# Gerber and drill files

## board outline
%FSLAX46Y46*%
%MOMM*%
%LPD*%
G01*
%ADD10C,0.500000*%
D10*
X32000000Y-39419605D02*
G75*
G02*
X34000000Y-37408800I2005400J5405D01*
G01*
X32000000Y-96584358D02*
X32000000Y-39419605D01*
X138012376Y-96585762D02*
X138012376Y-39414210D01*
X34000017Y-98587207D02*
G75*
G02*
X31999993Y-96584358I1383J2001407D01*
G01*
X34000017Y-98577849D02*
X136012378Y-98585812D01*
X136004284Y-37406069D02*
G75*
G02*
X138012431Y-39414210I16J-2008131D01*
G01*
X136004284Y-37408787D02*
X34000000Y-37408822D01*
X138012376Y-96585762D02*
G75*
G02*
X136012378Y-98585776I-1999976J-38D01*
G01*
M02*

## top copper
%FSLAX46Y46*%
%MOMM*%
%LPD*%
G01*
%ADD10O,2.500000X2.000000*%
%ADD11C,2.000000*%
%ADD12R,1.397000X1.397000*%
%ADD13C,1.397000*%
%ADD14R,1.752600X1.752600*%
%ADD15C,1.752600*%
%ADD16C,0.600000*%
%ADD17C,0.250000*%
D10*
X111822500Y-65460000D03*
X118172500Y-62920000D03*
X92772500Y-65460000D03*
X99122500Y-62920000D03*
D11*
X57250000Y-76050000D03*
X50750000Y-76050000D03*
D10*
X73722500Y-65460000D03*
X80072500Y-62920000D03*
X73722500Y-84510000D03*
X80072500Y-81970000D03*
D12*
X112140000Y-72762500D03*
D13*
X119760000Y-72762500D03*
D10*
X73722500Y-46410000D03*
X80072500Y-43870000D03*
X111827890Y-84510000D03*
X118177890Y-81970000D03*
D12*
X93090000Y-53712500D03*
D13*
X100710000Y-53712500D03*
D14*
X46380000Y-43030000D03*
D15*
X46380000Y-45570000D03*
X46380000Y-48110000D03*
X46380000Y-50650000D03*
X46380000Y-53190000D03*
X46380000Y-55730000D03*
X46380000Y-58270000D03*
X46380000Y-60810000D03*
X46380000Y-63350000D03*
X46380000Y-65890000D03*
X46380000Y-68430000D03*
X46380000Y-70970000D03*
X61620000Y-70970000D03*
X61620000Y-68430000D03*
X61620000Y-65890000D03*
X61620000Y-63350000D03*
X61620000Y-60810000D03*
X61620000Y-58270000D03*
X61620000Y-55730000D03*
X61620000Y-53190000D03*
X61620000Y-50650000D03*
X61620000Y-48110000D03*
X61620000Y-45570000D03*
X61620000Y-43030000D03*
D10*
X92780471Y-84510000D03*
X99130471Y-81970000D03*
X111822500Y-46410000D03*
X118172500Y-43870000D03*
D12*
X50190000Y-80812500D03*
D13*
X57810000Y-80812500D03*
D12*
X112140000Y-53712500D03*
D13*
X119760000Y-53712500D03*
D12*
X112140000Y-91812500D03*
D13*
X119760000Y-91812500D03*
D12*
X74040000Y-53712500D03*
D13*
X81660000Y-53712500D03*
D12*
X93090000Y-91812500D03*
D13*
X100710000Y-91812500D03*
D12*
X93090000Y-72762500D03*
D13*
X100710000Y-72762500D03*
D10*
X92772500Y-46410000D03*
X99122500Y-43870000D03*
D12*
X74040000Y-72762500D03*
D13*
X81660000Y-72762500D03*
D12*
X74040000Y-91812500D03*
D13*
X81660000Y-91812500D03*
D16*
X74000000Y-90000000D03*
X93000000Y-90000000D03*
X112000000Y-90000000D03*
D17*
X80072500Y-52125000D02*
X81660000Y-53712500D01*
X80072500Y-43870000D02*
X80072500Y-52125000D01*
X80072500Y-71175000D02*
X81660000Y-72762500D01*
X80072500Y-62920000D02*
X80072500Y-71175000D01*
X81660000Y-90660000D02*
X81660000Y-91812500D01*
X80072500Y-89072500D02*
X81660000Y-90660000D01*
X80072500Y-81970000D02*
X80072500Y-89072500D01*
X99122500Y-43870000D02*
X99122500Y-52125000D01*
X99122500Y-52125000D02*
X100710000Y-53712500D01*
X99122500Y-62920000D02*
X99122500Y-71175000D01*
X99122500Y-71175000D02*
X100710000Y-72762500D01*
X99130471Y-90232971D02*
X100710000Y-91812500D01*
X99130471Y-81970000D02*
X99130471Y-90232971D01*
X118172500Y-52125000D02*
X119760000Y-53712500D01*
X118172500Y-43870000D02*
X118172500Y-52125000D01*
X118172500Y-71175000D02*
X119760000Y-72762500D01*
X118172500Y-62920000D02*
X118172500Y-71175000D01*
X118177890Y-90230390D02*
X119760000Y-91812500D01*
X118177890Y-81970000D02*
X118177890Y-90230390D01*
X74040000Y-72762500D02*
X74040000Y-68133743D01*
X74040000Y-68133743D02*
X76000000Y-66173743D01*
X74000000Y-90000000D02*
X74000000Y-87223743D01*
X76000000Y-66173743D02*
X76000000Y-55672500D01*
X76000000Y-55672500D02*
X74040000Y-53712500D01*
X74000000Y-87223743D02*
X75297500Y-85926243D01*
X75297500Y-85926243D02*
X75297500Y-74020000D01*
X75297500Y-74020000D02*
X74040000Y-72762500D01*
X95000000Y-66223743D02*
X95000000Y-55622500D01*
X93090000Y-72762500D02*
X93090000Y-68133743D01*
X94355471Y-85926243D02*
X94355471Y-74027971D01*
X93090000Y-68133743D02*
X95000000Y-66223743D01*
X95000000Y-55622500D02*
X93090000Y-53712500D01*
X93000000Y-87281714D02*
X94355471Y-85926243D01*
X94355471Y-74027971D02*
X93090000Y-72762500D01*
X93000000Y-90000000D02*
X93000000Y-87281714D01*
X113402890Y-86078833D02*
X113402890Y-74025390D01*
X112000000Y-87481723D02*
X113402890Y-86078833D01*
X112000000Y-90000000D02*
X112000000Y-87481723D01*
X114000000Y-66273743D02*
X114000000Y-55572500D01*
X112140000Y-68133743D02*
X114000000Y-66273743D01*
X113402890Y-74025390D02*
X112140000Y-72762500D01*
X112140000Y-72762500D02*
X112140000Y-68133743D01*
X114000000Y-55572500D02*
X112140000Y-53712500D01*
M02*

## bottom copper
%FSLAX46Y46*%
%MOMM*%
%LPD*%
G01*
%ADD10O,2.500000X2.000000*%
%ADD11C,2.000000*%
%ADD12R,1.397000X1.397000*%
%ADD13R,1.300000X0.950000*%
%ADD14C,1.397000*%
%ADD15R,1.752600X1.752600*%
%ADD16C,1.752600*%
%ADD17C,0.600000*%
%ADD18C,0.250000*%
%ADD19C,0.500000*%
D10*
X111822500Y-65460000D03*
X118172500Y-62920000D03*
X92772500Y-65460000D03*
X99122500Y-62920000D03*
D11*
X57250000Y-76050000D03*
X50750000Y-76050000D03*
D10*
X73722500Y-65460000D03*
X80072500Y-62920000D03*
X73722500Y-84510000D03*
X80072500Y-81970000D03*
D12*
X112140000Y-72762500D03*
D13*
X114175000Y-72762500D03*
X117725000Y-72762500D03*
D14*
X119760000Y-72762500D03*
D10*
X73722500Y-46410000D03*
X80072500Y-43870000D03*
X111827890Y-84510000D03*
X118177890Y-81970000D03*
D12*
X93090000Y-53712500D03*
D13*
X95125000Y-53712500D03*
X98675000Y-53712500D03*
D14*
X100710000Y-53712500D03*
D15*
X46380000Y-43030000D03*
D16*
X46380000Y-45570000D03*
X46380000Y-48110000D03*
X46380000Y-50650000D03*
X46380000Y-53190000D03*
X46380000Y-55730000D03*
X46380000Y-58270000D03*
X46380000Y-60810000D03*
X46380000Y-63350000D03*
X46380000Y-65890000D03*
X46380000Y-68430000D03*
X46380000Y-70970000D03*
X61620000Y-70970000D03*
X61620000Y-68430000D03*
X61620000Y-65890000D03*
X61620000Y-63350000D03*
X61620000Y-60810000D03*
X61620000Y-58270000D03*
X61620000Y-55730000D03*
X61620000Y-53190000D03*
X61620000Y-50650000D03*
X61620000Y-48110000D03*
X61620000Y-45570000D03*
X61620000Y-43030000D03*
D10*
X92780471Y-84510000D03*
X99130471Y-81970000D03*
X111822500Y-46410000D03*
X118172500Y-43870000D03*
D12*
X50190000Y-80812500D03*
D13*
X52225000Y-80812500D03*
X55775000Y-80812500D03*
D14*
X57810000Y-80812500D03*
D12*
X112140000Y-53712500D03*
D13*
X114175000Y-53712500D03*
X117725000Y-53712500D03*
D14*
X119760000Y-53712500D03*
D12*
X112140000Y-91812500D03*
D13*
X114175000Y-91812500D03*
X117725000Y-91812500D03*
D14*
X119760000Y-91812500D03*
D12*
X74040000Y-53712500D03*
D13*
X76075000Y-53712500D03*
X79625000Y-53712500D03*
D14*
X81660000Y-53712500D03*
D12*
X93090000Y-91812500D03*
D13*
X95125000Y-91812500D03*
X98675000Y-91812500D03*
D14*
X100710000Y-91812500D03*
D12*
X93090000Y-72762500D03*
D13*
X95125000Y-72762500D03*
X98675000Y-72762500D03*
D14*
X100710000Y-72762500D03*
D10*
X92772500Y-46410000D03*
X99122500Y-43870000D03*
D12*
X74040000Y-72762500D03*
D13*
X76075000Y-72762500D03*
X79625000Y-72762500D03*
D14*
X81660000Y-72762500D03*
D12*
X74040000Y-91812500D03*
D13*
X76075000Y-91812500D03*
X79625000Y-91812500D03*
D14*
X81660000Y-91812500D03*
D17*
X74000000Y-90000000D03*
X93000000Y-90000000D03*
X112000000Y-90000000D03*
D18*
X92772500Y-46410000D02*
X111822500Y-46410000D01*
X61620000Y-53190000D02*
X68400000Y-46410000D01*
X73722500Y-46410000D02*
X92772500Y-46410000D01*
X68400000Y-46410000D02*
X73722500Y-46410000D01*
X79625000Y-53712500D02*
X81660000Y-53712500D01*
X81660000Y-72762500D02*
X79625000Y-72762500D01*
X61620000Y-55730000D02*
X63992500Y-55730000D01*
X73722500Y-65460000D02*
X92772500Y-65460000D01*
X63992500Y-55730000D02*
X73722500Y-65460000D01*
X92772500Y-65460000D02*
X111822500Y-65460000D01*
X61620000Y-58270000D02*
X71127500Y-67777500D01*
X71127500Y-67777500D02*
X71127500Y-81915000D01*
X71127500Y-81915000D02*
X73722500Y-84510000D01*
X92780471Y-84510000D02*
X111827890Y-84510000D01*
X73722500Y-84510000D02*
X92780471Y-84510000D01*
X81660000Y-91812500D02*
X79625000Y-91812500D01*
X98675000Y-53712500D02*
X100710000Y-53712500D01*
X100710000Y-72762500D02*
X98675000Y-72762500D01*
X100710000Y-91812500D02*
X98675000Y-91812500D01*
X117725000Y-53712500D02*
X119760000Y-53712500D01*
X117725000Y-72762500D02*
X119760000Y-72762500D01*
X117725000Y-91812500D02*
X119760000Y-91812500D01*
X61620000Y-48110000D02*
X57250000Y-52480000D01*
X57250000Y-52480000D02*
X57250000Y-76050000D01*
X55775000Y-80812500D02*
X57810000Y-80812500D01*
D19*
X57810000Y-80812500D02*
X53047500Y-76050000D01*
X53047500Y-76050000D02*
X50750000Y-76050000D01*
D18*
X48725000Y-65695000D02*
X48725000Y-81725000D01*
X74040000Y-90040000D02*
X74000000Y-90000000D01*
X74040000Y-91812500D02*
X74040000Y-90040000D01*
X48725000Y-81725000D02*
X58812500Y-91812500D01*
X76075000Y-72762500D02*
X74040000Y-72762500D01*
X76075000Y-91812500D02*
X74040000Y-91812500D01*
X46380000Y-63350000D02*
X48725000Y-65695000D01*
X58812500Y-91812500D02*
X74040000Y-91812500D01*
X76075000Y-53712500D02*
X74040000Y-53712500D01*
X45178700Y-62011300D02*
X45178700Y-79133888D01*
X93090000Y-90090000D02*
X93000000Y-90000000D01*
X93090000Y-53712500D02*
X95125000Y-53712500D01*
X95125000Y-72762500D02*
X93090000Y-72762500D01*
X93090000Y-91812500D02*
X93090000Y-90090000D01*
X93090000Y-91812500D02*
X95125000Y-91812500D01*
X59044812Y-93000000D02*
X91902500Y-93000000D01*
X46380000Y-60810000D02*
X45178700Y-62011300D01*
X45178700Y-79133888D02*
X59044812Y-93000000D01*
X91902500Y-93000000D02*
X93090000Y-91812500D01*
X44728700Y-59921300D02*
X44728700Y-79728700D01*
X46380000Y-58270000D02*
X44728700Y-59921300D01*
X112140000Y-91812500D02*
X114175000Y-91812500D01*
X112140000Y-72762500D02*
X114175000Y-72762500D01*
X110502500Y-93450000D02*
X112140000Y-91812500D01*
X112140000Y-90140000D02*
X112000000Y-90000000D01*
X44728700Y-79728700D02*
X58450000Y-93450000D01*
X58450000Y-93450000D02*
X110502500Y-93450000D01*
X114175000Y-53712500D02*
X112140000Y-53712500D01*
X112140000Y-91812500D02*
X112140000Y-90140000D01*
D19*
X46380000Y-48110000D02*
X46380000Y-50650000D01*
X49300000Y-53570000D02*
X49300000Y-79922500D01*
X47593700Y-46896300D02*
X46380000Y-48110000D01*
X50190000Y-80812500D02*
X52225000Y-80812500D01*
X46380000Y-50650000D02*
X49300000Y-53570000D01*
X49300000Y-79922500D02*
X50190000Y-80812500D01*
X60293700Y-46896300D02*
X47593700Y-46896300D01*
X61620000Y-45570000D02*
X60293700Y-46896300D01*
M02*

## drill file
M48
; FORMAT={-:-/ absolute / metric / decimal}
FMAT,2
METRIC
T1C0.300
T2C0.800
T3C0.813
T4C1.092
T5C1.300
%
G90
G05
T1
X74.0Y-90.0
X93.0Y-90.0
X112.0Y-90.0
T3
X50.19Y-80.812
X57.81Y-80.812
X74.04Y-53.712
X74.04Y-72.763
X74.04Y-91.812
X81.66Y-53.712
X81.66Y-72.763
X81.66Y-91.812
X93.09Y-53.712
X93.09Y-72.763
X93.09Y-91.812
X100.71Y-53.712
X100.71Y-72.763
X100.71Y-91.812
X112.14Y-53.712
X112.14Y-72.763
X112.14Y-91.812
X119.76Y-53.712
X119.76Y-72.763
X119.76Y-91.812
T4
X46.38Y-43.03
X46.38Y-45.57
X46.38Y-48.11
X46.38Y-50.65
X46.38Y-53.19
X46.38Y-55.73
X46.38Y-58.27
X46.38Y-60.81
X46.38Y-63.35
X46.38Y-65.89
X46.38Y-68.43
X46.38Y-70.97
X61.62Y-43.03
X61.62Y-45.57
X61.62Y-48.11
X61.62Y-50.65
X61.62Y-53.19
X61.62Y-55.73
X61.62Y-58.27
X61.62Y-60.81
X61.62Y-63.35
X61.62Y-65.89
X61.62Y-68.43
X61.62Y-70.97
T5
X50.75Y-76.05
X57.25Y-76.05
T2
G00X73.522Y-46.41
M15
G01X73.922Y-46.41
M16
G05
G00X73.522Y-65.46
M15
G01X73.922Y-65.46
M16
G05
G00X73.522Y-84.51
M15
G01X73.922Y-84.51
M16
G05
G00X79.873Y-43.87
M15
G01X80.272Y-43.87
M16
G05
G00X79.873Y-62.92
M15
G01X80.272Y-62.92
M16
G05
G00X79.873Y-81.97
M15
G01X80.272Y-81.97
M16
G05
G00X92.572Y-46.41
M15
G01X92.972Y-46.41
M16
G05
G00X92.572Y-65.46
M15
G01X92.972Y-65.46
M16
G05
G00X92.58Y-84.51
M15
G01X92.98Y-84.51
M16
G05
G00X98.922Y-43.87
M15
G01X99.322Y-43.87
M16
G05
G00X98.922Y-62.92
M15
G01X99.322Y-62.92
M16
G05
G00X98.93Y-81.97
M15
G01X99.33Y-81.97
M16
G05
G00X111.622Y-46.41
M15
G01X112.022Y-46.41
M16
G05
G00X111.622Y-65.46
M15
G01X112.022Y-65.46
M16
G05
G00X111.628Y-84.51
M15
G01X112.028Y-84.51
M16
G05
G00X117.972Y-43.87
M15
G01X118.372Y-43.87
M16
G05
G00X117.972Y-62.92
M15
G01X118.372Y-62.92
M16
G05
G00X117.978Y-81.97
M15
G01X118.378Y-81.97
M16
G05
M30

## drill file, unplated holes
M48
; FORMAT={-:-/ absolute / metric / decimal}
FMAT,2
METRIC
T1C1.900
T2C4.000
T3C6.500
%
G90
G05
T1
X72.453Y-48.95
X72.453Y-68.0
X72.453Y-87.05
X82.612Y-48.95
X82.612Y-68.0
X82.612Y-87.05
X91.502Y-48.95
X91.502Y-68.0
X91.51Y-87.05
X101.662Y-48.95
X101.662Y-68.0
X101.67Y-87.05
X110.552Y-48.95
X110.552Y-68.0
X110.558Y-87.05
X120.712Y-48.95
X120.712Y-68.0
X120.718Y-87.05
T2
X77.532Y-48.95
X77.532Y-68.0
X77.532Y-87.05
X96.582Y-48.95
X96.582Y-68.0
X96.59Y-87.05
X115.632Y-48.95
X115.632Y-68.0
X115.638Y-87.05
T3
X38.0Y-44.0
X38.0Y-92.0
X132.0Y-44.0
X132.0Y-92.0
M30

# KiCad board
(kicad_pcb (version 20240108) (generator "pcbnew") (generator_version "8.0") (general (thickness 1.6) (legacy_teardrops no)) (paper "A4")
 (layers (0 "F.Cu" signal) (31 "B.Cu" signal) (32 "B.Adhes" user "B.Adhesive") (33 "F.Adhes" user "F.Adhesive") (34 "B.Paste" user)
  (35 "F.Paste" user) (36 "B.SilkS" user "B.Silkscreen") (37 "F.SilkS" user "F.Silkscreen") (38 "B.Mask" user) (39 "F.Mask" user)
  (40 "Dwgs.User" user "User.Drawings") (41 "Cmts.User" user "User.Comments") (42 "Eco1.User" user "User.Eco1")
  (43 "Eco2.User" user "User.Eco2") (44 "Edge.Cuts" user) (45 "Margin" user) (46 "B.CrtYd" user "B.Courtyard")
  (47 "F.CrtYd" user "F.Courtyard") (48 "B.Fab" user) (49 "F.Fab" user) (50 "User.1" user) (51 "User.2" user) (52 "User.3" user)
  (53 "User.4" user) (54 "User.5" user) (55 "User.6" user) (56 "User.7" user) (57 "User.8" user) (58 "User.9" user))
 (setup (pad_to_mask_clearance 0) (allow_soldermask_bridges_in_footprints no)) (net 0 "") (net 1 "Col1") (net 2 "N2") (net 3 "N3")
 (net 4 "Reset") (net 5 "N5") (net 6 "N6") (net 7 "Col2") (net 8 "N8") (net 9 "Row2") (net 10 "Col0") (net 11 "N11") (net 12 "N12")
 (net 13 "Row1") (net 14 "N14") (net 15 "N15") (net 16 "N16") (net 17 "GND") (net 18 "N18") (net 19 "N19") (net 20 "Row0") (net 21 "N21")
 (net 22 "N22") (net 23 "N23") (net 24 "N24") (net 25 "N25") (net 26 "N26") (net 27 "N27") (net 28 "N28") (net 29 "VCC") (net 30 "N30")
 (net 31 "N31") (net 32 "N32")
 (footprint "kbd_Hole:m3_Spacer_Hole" (layer "F.Cu") (at 38 92)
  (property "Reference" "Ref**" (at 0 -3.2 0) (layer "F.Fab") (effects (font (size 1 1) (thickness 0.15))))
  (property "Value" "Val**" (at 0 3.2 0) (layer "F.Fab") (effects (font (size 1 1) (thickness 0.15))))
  (pad "" np_thru_hole circle (at 0 0) (size 6.5 6.5) (drill 6.5) (layers "*.Cu" "*.Mask")))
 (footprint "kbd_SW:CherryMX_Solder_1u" (layer "F.Cu") (at 115.6325 68)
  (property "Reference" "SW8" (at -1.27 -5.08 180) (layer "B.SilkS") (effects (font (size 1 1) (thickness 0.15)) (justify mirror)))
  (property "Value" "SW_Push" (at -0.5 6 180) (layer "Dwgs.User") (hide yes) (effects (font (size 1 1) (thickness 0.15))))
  (pad "" np_thru_hole circle (at -5.08 0 90) (size 1.9 1.9) (drill 1.9) (layers "*.Cu" "*.Mask"))
  (pad "" np_thru_hole circle (at 0 0 90) (size 4 4) (drill 4) (layers "*.Cu" "*.Mask"))
  (pad "" np_thru_hole circle (at 5.08 0 90) (size 1.9 1.9) (drill 1.9) (layers "*.Cu" "*.Mask"))
  (pad "1" thru_hole oval (at -3.81 -2.54) (size 2.5 2) (drill oval 1.2 0.8) (layers "*.Cu" "F.SilkS" "B.Mask") (remove_unused_layers no)
   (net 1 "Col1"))
  (pad "2" thru_hole oval (at 2.54 -5.08) (size 2.5 2) (drill oval 1.2 0.8) (layers "*.Cu" "F.SilkS" "B.Mask") (remove_unused_layers no)
   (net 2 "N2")))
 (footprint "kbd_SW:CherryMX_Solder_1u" (layer "F.Cu") (at 96.5825 68)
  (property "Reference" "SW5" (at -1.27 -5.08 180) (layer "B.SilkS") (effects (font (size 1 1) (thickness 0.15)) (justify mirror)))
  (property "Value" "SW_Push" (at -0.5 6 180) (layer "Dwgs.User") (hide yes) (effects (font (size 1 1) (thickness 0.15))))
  (pad "" np_thru_hole circle (at -5.08 0 90) (size 1.9 1.9) (drill 1.9) (layers "*.Cu" "*.Mask"))
  (pad "" np_thru_hole circle (at 0 0 90) (size 4 4) (drill 4) (layers "*.Cu" "*.Mask"))
  (pad "" np_thru_hole circle (at 5.08 0 90) (size 1.9 1.9) (drill 1.9) (layers "*.Cu" "*.Mask"))
  (pad "1" thru_hole oval (at -3.81 -2.54) (size 2.5 2) (drill oval 1.2 0.8) (layers "*.Cu" "F.SilkS" "B.Mask") (remove_unused_layers no)
   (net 1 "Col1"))
  (pad "2" thru_hole oval (at 2.54 -5.08) (size 2.5 2) (drill oval 1.2 0.8) (layers "*.Cu" "F.SilkS" "B.Mask") (remove_unused_layers no)
   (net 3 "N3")))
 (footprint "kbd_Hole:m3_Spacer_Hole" (layer "F.Cu") (at 132 92)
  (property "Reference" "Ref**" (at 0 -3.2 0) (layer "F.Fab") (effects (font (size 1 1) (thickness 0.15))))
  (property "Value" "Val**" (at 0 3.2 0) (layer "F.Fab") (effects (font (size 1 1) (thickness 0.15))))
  (pad "" np_thru_hole circle (at 0 0) (size 6.5 6.5) (drill 6.5) (layers "*.Cu" "*.Mask")))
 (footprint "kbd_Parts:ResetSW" (layer "F.Cu") (at 54 76.05)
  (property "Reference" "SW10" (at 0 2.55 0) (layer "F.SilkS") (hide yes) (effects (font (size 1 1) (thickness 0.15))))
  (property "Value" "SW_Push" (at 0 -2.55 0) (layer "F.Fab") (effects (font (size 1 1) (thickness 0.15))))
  (pad "1" thru_hole circle (at 3.25 0) (size 2 2) (drill 1.3) (layers "*.Cu" "*.Mask" "F.SilkS") (remove_unused_layers no) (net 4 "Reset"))
  (pad "2" thru_hole circle (at -3.25 0) (size 2 2) (drill 1.3) (layers "*.Cu" "*.Mask" "F.SilkS") (remove_unused_layers no) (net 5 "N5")))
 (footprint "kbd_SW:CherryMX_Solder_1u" (layer "F.Cu") (at 77.5325 68)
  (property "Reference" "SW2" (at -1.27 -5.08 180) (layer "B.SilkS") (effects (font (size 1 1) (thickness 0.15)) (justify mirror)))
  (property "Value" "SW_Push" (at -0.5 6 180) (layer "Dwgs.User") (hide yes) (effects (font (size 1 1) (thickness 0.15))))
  (pad "" np_thru_hole circle (at -5.08 0 90) (size 1.9 1.9) (drill 1.9) (layers "*.Cu" "*.Mask"))
  (pad "" np_thru_hole circle (at 0 0 90) (size 4 4) (drill 4) (layers "*.Cu" "*.Mask"))
  (pad "" np_thru_hole circle (at 5.08 0 90) (size 1.9 1.9) (drill 1.9) (layers "*.Cu" "*.Mask"))
  (pad "1" thru_hole oval (at -3.81 -2.54) (size 2.5 2) (drill oval 1.2 0.8) (layers "*.Cu" "F.SilkS" "B.Mask") (remove_unused_layers no)
   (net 1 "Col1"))
  (pad "2" thru_hole oval (at 2.54 -5.08) (size 2.5 2) (drill oval 1.2 0.8) (layers "*.Cu" "F.SilkS" "B.Mask") (remove_unused_layers no)
   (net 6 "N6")))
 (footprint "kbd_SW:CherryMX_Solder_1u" (layer "F.Cu") (at 77.5325 87.05)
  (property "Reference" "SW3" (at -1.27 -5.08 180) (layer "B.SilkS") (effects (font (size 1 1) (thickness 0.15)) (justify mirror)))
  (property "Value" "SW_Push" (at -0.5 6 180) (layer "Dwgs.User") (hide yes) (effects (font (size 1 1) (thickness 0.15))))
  (pad "" np_thru_hole circle (at -5.08 0 90) (size 1.9 1.9) (drill 1.9) (layers "*.Cu" "*.Mask"))
  (pad "" np_thru_hole circle (at 0 0 90) (size 4 4) (drill 4) (layers "*.Cu" "*.Mask"))
  (pad "" np_thru_hole circle (at 5.08 0 90) (size 1.9 1.9) (drill 1.9) (layers "*.Cu" "*.Mask"))
  (pad "1" thru_hole oval (at -3.81 -2.54) (size 2.5 2) (drill oval 1.2 0.8) (layers "*.Cu" "F.SilkS" "B.Mask") (remove_unused_layers no)
   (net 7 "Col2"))
  (pad "2" thru_hole oval (at 2.54 -5.08) (size 2.5 2) (drill oval 1.2 0.8) (layers "*.Cu" "F.SilkS" "B.Mask") (remove_unused_layers no)
   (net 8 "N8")))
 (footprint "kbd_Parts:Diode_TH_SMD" (layer "F.Cu") (at 115.95 72.7625)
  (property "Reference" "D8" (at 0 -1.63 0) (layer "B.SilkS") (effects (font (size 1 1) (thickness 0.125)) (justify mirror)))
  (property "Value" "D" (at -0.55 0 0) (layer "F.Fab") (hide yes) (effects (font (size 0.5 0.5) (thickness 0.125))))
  (pad "1" thru_hole rect (at -3.81 0) (size 1.397 1.397) (drill 0.8128) (layers "*.Cu" "*.Mask" "F.SilkS") (remove_unused_layers no)
   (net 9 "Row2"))
  (pad "1" smd rect (at -1.775 0) (size 1.3 0.95) (layers "B.Cu" "B.Paste" "B.Mask") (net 9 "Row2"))
  (pad "2" smd rect (at 1.775 0) (size 1.3 0.95) (layers "B.Cu" "B.Paste" "B.Mask") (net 2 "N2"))
  (pad "2" thru_hole circle (at 3.81 0) (size 1.397 1.397) (drill 0.8128) (layers "*.Cu" "*.Mask" "F.SilkS") (remove_unused_layers no)
   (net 2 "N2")))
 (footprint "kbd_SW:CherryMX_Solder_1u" (layer "F.Cu") (at 77.5325 48.95)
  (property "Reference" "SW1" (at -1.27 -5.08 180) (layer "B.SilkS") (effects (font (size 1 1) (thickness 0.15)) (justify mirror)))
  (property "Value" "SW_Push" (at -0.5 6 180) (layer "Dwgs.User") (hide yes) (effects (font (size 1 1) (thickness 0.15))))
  (pad "" np_thru_hole circle (at -5.08 0 90) (size 1.9 1.9) (drill 1.9) (layers "*.Cu" "*.Mask"))
  (pad "" np_thru_hole circle (at 0 0 90) (size 4 4) (drill 4) (layers "*.Cu" "*.Mask"))
  (pad "" np_thru_hole circle (at 5.08 0 90) (size 1.9 1.9) (drill 1.9) (layers "*.Cu" "*.Mask"))
  (pad "1" thru_hole oval (at -3.81 -2.54) (size 2.5 2) (drill oval 1.2 0.8) (layers "*.Cu" "F.SilkS" "B.Mask") (remove_unused_layers no)
   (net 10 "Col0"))
  (pad "2" thru_hole oval (at 2.54 -5.08) (size 2.5 2) (drill oval 1.2 0.8) (layers "*.Cu" "F.SilkS" "B.Mask") (remove_unused_layers no)
   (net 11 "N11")))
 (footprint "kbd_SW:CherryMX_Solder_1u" (layer "F.Cu") (at 115.63789 87.05)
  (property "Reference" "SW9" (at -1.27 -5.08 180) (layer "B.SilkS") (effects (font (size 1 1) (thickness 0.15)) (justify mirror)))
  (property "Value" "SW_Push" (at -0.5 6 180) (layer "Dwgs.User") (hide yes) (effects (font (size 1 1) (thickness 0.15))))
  (pad "" np_thru_hole circle (at -5.08 0 90) (size 1.9 1.9) (drill 1.9) (layers "*.Cu" "*.Mask"))
  (pad "" np_thru_hole circle (at 0 0 90) (size 4 4) (drill 4) (layers "*.Cu" "*.Mask"))
  (pad "" np_thru_hole circle (at 5.08 0 90) (size 1.9 1.9) (drill 1.9) (layers "*.Cu" "*.Mask"))
  (pad "1" thru_hole oval (at -3.81 -2.54) (size 2.5 2) (drill oval 1.2 0.8) (layers "*.Cu" "F.SilkS" "B.Mask") (remove_unused_layers no)
   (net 7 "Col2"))
  (pad "2" thru_hole oval (at 2.54 -5.08) (size 2.5 2) (drill oval 1.2 0.8) (layers "*.Cu" "F.SilkS" "B.Mask") (remove_unused_layers no)
   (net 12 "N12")))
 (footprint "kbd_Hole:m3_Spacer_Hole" (layer "F.Cu") (at 132 44)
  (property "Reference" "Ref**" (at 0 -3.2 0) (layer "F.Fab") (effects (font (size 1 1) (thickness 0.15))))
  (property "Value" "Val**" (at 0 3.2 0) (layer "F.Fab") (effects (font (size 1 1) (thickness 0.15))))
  (pad "" np_thru_hole circle (at 0 0) (size 6.5 6.5) (drill 6.5) (layers "*.Cu" "*.Mask")))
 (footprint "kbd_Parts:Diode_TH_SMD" (layer "F.Cu") (at 96.9 53.7125)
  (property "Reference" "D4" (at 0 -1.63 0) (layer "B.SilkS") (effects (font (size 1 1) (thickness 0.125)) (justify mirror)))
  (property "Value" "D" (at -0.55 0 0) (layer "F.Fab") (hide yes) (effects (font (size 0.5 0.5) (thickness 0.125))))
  (pad "1" thru_hole rect (at -3.81 0) (size 1.397 1.397) (drill 0.8128) (layers "*.Cu" "*.Mask" "F.SilkS") (remove_unused_layers no)
   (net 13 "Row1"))
  (pad "1" smd rect (at -1.775 0) (size 1.3 0.95) (layers "B.Cu" "B.Paste" "B.Mask") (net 13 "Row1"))
  (pad "2" smd rect (at 1.775 0) (size 1.3 0.95) (layers "B.Cu" "B.Paste" "B.Mask") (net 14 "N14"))
  (pad "2" thru_hole circle (at 3.81 0) (size 1.397 1.397) (drill 0.8128) (layers "*.Cu" "*.Mask" "F.SilkS") (remove_unused_layers no)
   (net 14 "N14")))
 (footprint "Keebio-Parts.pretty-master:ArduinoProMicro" (layer "F.Cu") (at 54 57 -90)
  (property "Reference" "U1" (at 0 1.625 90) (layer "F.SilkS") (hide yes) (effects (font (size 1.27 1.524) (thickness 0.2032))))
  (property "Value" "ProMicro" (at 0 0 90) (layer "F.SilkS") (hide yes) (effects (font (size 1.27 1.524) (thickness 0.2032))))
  (pad "1" thru_hole rect (at -13.97 7.62 270) (size 1.7526 1.7526) (drill 1.0922) (layers "*.Cu" "*.SilkS" "*.Mask")
   (remove_unused_layers no) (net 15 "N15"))
  (pad "2" thru_hole circle (at -11.43 7.62 270) (size 1.7526 1.7526) (drill 1.0922) (layers "*.Cu" "*.SilkS" "*.Mask")
   (remove_unused_layers no) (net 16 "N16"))
  (pad "3" thru_hole circle (at -8.89 7.62 270) (size 1.7526 1.7526) (drill 1.0922) (layers "*.Cu" "*.SilkS" "*.Mask")
   (remove_unused_layers no) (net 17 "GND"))
  (pad "4" thru_hole circle (at -6.35 7.62 270) (size 1.7526 1.7526) (drill 1.0922) (layers "*.Cu" "*.SilkS" "*.Mask")
   (remove_unused_layers no) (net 17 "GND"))
  (pad "5" thru_hole circle (at -3.81 7.62 270) (size 1.7526 1.7526) (drill 1.0922) (layers "*.Cu" "*.SilkS" "*.Mask")
   (remove_unused_layers no) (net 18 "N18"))
  (pad "6" thru_hole circle (at -1.27 7.62 270) (size 1.7526 1.7526) (drill 1.0922) (layers "*.Cu" "*.SilkS" "*.Mask")
   (remove_unused_layers no) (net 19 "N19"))
  (pad "7" thru_hole circle (at 1.27 7.62 270) (size 1.7526 1.7526) (drill 1.0922) (layers "*.Cu" "*.SilkS" "*.Mask")
   (remove_unused_layers no) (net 9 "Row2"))
  (pad "8" thru_hole circle (at 3.81 7.62 270) (size 1.7526 1.7526) (drill 1.0922) (layers "*.Cu" "*.SilkS" "*.Mask")
   (remove_unused_layers no) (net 13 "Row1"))
  (pad "9" thru_hole circle (at 6.35 7.62 270) (size 1.7526 1.7526) (drill 1.0922) (layers "*.Cu" "*.SilkS" "*.Mask")
   (remove_unused_layers no) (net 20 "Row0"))
  (pad "10" thru_hole circle (at 8.89 7.62 270) (size 1.7526 1.7526) (drill 1.0922) (layers "*.Cu" "*.SilkS" "*.Mask")
   (remove_unused_layers no) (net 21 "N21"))
  (pad "11" thru_hole circle (at 11.43 7.62 270) (size 1.7526 1.7526) (drill 1.0922) (layers "*.Cu" "*.SilkS" "*.Mask")
   (remove_unused_layers no) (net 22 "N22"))
  (pad "12" thru_hole circle (at 13.97 7.62 270) (size 1.7526 1.7526) (drill 1.0922) (layers "*.Cu" "*.SilkS" "*.Mask")
   (remove_unused_layers no) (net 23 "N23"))
  (pad "13" thru_hole circle (at 13.97 -7.62 270) (size 1.7526 1.7526) (drill 1.0922) (layers "*.Cu" "*.SilkS" "*.Mask")
   (remove_unused_layers no) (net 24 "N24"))
  (pad "14" thru_hole circle (at 11.43 -7.62 270) (size 1.7526 1.7526) (drill 1.0922) (layers "*.Cu" "*.SilkS" "*.Mask")
   (remove_unused_layers no) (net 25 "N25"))
  (pad "15" thru_hole circle (at 8.89 -7.62 270) (size 1.7526 1.7526) (drill 1.0922) (layers "*.Cu" "*.SilkS" "*.Mask")
   (remove_unused_layers no) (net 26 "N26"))
  (pad "16" thru_hole circle (at 6.35 -7.62 270) (size 1.7526 1.7526) (drill 1.0922) (layers "*.Cu" "*.SilkS" "*.Mask")
   (remove_unused_layers no) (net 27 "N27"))
  (pad "17" thru_hole circle (at 3.81 -7.62 270) (size 1.7526 1.7526) (drill 1.0922) (layers "*.Cu" "*.SilkS" "*.Mask")
   (remove_unused_layers no) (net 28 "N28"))
  (pad "18" thru_hole circle (at 1.27 -7.62 270) (size 1.7526 1.7526) (drill 1.0922) (layers "*.Cu" "*.SilkS" "*.Mask")
   (remove_unused_layers no) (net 7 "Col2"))
  (pad "19" thru_hole circle (at -1.27 -7.62 270) (size 1.7526 1.7526) (drill 1.0922) (layers "*.Cu" "*.SilkS" "*.Mask")
   (remove_unused_layers no) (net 1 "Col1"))
  (pad "20" thru_hole circle (at -3.81 -7.62 270) (size 1.7526 1.7526) (drill 1.0922) (layers "*.Cu" "*.SilkS" "*.Mask")
   (remove_unused_layers no) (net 10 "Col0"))
  (pad "21" thru_hole circle (at -6.35 -7.62 270) (size 1.7526 1.7526) (drill 1.0922) (layers "*.Cu" "*.SilkS" "*.Mask")
   (remove_unused_layers no) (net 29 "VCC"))
  (pad "22" thru_hole circle (at -8.89 -7.62 270) (size 1.7526 1.7526) (drill 1.0922) (layers "*.Cu" "*.SilkS" "*.Mask")
   (remove_unused_layers no) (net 4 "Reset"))
  (pad "23" thru_hole circle (at -11.43 -7.62 270) (size 1.7526 1.7526) (drill 1.0922) (layers "*.Cu" "*.SilkS" "*.Mask")
   (remove_unused_layers no) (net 17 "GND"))
  (pad "24" thru_hole circle (at -13.97 -7.62 270) (size 1.7526 1.7526) (drill 1.0922) (layers "*.Cu" "*.SilkS" "*.Mask")
   (remove_unused_layers no) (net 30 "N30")))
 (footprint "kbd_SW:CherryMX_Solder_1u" (layer "F.Cu") (at 96.590471 87.05)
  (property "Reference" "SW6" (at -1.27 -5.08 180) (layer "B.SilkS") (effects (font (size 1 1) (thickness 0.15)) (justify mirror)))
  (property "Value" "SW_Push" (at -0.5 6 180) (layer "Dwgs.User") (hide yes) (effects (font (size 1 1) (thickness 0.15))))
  (pad "" np_thru_hole circle (at -5.08 0 90) (size 1.9 1.9) (drill 1.9) (layers "*.Cu" "*.Mask"))
  (pad "" np_thru_hole circle (at 0 0 90) (size 4 4) (drill 4) (layers "*.Cu" "*.Mask"))
  (pad "" np_thru_hole circle (at 5.08 0 90) (size 1.9 1.9) (drill 1.9) (layers "*.Cu" "*.Mask"))
  (pad "1" thru_hole oval (at -3.81 -2.54) (size 2.5 2) (drill oval 1.2 0.8) (layers "*.Cu" "F.SilkS" "B.Mask") (remove_unused_layers no)
   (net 7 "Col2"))
  (pad "2" thru_hole oval (at 2.54 -5.08) (size 2.5 2) (drill oval 1.2 0.8) (layers "*.Cu" "F.SilkS" "B.Mask") (remove_unused_layers no)
   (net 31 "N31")))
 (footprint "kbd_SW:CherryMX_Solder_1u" (layer "F.Cu") (at 115.6325 48.95)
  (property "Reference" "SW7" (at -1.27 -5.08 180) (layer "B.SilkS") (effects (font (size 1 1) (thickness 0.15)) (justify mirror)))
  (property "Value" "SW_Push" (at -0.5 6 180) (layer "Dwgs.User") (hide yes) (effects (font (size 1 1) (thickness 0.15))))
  (pad "" np_thru_hole circle (at -5.08 0 90) (size 1.9 1.9) (drill 1.9) (layers "*.Cu" "*.Mask"))
  (pad "" np_thru_hole circle (at 0 0 90) (size 4 4) (drill 4) (layers "*.Cu" "*.Mask"))
  (pad "" np_thru_hole circle (at 5.08 0 90) (size 1.9 1.9) (drill 1.9) (layers "*.Cu" "*.Mask"))
  (pad "1" thru_hole oval (at -3.81 -2.54) (size 2.5 2) (drill oval 1.2 0.8) (layers "*.Cu" "F.SilkS" "B.Mask") (remove_unused_layers no)
   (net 10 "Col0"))
  (pad "2" thru_hole oval (at 2.54 -5.08) (size 2.5 2) (drill oval 1.2 0.8) (layers "*.Cu" "F.SilkS" "B.Mask") (remove_unused_layers no)
   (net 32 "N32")))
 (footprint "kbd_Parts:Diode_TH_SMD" (layer "F.Cu") (at 54 80.8125)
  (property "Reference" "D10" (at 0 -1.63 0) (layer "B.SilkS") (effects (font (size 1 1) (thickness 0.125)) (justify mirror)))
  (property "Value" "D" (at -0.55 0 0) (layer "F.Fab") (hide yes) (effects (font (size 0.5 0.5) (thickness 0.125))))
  (pad "1" thru_hole rect (at -3.81 0) (size 1.397 1.397) (drill 0.8128) (layers "*.Cu" "*.Mask" "F.SilkS") (remove_unused_layers no)
   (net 17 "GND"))
  (pad "1" smd rect (at -1.775 0) (size 1.3 0.95) (layers "B.Cu" "B.Paste" "B.Mask") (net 17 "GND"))
  (pad "2" smd rect (at 1.775 0) (size 1.3 0.95) (layers "B.Cu" "B.Paste" "B.Mask") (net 5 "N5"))
  (pad "2" thru_hole circle (at 3.81 0) (size 1.397 1.397) (drill 0.8128) (layers "*.Cu" "*.Mask" "F.SilkS") (remove_unused_layers no)
   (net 5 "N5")))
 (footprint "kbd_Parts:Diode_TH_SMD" (layer "F.Cu") (at 115.95 53.7125)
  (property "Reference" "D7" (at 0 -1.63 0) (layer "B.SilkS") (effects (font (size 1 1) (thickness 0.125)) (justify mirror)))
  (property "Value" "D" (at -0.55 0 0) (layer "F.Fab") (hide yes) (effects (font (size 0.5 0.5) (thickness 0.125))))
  (pad "1" thru_hole rect (at -3.81 0) (size 1.397 1.397) (drill 0.8128) (layers "*.Cu" "*.Mask" "F.SilkS") (remove_unused_layers no)
   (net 9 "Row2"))
  (pad "1" smd rect (at -1.775 0) (size 1.3 0.95) (layers "B.Cu" "B.Paste" "B.Mask") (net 9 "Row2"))
  (pad "2" smd rect (at 1.775 0) (size 1.3 0.95) (layers "B.Cu" "B.Paste" "B.Mask") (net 32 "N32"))
  (pad "2" thru_hole circle (at 3.81 0) (size 1.397 1.397) (drill 0.8128) (layers "*.Cu" "*.Mask" "F.SilkS") (remove_unused_layers no)
   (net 32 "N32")))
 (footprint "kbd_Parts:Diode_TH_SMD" (layer "F.Cu") (at 115.95 91.8125)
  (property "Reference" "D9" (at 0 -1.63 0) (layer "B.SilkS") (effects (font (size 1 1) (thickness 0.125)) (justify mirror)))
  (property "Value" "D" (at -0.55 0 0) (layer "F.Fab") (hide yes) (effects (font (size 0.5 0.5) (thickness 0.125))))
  (pad "1" thru_hole rect (at -3.81 0) (size 1.397 1.397) (drill 0.8128) (layers "*.Cu" "*.Mask" "F.SilkS") (remove_unused_layers no)
   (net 9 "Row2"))
  (pad "1" smd rect (at -1.775 0) (size 1.3 0.95) (layers "B.Cu" "B.Paste" "B.Mask") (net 9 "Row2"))
  (pad "2" smd rect (at 1.775 0) (size 1.3 0.95) (layers "B.Cu" "B.Paste" "B.Mask") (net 12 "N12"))
  (pad "2" thru_hole circle (at 3.81 0) (size 1.397 1.397) (drill 0.8128) (layers "*.Cu" "*.Mask" "F.SilkS") (remove_unused_layers no)
   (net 12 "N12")))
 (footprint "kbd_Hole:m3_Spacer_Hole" (layer "F.Cu") (at 38 44)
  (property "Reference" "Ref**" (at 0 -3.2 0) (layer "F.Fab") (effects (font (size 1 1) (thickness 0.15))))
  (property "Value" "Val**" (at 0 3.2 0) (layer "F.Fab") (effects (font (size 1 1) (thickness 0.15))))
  (pad "" np_thru_hole circle (at 0 0) (size 6.5 6.5) (drill 6.5) (layers "*.Cu" "*.Mask")))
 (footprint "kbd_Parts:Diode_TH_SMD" (layer "F.Cu") (at 77.85 53.7125)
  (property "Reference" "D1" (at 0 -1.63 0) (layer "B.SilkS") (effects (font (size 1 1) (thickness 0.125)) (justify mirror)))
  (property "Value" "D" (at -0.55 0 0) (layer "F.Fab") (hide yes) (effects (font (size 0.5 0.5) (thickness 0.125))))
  (pad "1" thru_hole rect (at -3.81 0) (size 1.397 1.397) (drill 0.8128) (layers "*.Cu" "*.Mask" "F.SilkS") (remove_unused_layers no)
   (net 20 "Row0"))
  (pad "1" smd rect (at -1.775 0) (size 1.3 0.95) (layers "B.Cu" "B.Paste" "B.Mask") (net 20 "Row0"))
  (pad "2" smd rect (at 1.775 0) (size 1.3 0.95) (layers "B.Cu" "B.Paste" "B.Mask") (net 11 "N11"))
  (pad "2" thru_hole circle (at 3.81 0) (size 1.397 1.397) (drill 0.8128) (layers "*.Cu" "*.Mask" "F.SilkS") (remove_unused_layers no)
   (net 11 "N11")))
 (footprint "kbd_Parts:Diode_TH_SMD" (layer "F.Cu") (at 96.9 91.8125)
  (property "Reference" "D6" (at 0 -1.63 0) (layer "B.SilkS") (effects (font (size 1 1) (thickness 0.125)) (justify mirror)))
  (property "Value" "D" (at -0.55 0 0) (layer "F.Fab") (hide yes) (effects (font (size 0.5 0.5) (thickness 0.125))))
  (pad "1" thru_hole rect (at -3.81 0) (size 1.397 1.397) (drill 0.8128) (layers "*.Cu" "*.Mask" "F.SilkS") (remove_unused_layers no)
   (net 13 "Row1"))
  (pad "1" smd rect (at -1.775 0) (size 1.3 0.95) (layers "B.Cu" "B.Paste" "B.Mask") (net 13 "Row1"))
  (pad "2" smd rect (at 1.775 0) (size 1.3 0.95) (layers "B.Cu" "B.Paste" "B.Mask") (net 31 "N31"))
  (pad "2" thru_hole circle (at 3.81 0) (size 1.397 1.397) (drill 0.8128) (layers "*.Cu" "*.Mask" "F.SilkS") (remove_unused_layers no)
   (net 31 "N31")))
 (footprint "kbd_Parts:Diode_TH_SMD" (layer "F.Cu") (at 96.9 72.7625)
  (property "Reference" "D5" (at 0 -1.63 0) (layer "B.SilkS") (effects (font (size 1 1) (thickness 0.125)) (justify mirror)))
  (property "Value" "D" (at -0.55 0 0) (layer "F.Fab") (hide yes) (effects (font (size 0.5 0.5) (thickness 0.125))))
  (pad "1" thru_hole rect (at -3.81 0) (size 1.397 1.397) (drill 0.8128) (layers "*.Cu" "*.Mask" "F.SilkS") (remove_unused_layers no)
   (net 13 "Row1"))
  (pad "1" smd rect (at -1.775 0) (size 1.3 0.95) (layers "B.Cu" "B.Paste" "B.Mask") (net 13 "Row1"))
  (pad "2" smd rect (at 1.775 0) (size 1.3 0.95) (layers "B.Cu" "B.Paste" "B.Mask") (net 3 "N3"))
  (pad "2" thru_hole circle (at 3.81 0) (size 1.397 1.397) (drill 0.8128) (layers "*.Cu" "*.Mask" "F.SilkS") (remove_unused_layers no)
   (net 3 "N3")))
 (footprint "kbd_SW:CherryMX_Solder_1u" (layer "F.Cu") (at 96.5825 48.95)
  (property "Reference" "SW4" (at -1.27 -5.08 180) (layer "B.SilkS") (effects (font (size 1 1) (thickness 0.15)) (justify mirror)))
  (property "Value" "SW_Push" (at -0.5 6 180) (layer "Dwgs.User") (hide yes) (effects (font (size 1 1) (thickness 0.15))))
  (pad "" np_thru_hole circle (at -5.08 0 90) (size 1.9 1.9) (drill 1.9) (layers "*.Cu" "*.Mask"))
  (pad "" np_thru_hole circle (at 0 0 90) (size 4 4) (drill 4) (layers "*.Cu" "*.Mask"))
  (pad "" np_thru_hole circle (at 5.08 0 90) (size 1.9 1.9) (drill 1.9) (layers "*.Cu" "*.Mask"))
  (pad "1" thru_hole oval (at -3.81 -2.54) (size 2.5 2) (drill oval 1.2 0.8) (layers "*.Cu" "F.SilkS" "B.Mask") (remove_unused_layers no)
   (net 10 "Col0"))
  (pad "2" thru_hole oval (at 2.54 -5.08) (size 2.5 2) (drill oval 1.2 0.8) (layers "*.Cu" "F.SilkS" "B.Mask") (remove_unused_layers no)
   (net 14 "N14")))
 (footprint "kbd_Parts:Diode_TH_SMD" (layer "F.Cu") (at 77.85 72.7625)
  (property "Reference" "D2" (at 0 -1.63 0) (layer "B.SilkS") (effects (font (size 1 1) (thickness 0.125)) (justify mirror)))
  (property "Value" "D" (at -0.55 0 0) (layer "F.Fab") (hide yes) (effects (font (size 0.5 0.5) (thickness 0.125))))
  (pad "1" thru_hole rect (at -3.81 0) (size 1.397 1.397) (drill 0.8128) (layers "*.Cu" "*.Mask" "F.SilkS") (remove_unused_layers no)
   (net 20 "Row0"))
  (pad "1" smd rect (at -1.775 0) (size 1.3 0.95) (layers "B.Cu" "B.Paste" "B.Mask") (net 20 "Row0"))
  (pad "2" smd rect (at 1.775 0) (size 1.3 0.95) (layers "B.Cu" "B.Paste" "B.Mask") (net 6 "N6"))
  (pad "2" thru_hole circle (at 3.81 0) (size 1.397 1.397) (drill 0.8128) (layers "*.Cu" "*.Mask" "F.SilkS") (remove_unused_layers no)
   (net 6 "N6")))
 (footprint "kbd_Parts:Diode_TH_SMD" (layer "F.Cu") (at 77.85 91.8125)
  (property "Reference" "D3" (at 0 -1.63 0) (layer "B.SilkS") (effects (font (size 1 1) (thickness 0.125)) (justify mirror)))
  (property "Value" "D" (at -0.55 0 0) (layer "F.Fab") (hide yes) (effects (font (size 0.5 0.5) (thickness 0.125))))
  (pad "1" thru_hole rect (at -3.81 0) (size 1.397 1.397) (drill 0.8128) (layers "*.Cu" "*.Mask" "F.SilkS") (remove_unused_layers no)
   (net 20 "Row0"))
  (pad "1" smd rect (at -1.775 0) (size 1.3 0.95) (layers "B.Cu" "B.Paste" "B.Mask") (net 20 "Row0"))
  (pad "2" smd rect (at 1.775 0) (size 1.3 0.95) (layers "B.Cu" "B.Paste" "B.Mask") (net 8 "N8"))
  (pad "2" thru_hole circle (at 3.81 0) (size 1.397 1.397) (drill 0.8128) (layers "*.Cu" "*.Mask" "F.SilkS") (remove_unused_layers no)
   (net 8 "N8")))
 (gr_arc (start 32 39.419605) (mid 32.583553 38) (end 34 37.408822) (stroke (width 0.5) (type default)) (layer "Edge.Cuts"))
 (gr_line (start 32 96.584358) (end 32 39.419605) (stroke (width 0.5) (type default)) (layer "Edge.Cuts"))
 (gr_line (start 138.012376 96.585762) (end 138.012376 39.41421) (stroke (width 0.5) (type default)) (layer "Edge.Cuts"))
 (gr_arc (start 34.000017 98.587207) (mid 32.585205 98) (end 32 96.584358) (stroke (width 0.5) (type default)) (layer "Edge.Cuts"))
 (gr_line (start 34.000017 98.577849) (end 136.012378 98.585812) (stroke (width 0.5) (type default)) (layer "Edge.Cuts"))
 (gr_arc (start 136.004284 37.406069) (mid 137.424229 37.99425) (end 138.012376 39.41421) (stroke (width 0.5) (type default))
  (layer "Edge.Cuts"))
 (gr_line (start 136.004284 37.408787) (end 34 37.408822) (stroke (width 0.5) (type default)) (layer "Edge.Cuts"))
 (gr_arc (start 138.012376 96.585762) (mid 137.426601 98) (end 136.012378 98.585812) (stroke (width 0.5) (type default)) (layer "Edge.Cuts"))
 (segment (start 92.7725 46.41) (end 111.8225 46.41) (width 0.25) (layer "B.Cu") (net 10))
 (segment (start 61.62 53.19) (end 68.4 46.41) (width 0.25) (layer "B.Cu") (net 10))
 (segment (start 73.7225 46.41) (end 92.7725 46.41) (width 0.25) (layer "B.Cu") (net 10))
 (segment (start 68.4 46.41) (end 73.7225 46.41) (width 0.25) (layer "B.Cu") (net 10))
 (segment (start 80.0725 52.125) (end 81.66 53.7125) (width 0.25) (layer "F.Cu") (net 11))
 (segment (start 80.0725 43.87) (end 80.0725 52.125) (width 0.25) (layer "F.Cu") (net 11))
 (segment (start 79.625 53.7125) (end 81.66 53.7125) (width 0.25) (layer "B.Cu") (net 11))
 (segment (start 80.0725 71.175) (end 81.66 72.7625) (width 0.25) (layer "F.Cu") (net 6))
 (segment (start 80.0725 62.92) (end 80.0725 71.175) (width 0.25) (layer "F.Cu") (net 6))
 (segment (start 81.66 72.7625) (end 79.625 72.7625) (width 0.25) (layer "B.Cu") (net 6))
 (segment (start 61.62 55.73) (end 63.9925 55.73) (width 0.25) (layer "B.Cu") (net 1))
 (segment (start 73.7225 65.46) (end 92.7725 65.46) (width 0.25) (layer "B.Cu") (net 1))
 (segment (start 63.9925 55.73) (end 73.7225 65.46) (width 0.25) (layer "B.Cu") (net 1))
 (segment (start 92.7725 65.46) (end 111.8225 65.46) (width 0.25) (layer "B.Cu") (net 1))
 (segment (start 61.62 58.27) (end 71.1275 67.7775) (width 0.25) (layer "B.Cu") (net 7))
 (segment (start 71.1275 67.7775) (end 71.1275 81.915) (width 0.25) (layer "B.Cu") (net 7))
 (segment (start 71.1275 81.915) (end 73.7225 84.51) (width 0.25) (layer "B.Cu") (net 7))
 (segment (start 92.780471 84.51) (end 111.82789 84.51) (width 0.25) (layer "B.Cu") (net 7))
 (segment (start 73.7225 84.51) (end 92.780471 84.51) (width 0.25) (layer "B.Cu") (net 7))
 (segment (start 81.66 90.66) (end 81.66 91.8125) (width 0.25) (layer "F.Cu") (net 8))
 (segment (start 80.0725 89.0725) (end 81.66 90.66) (width 0.25) (layer "F.Cu") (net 8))
 (segment (start 80.0725 81.97) (end 80.0725 89.0725) (width 0.25) (layer "F.Cu") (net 8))
 (segment (start 81.66 91.8125) (end 79.625 91.8125) (width 0.25) (layer "B.Cu") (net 8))
 (segment (start 99.1225 43.87) (end 99.1225 52.125) (width 0.25) (layer "F.Cu") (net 14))
 (segment (start 99.1225 52.125) (end 100.71 53.7125) (width 0.25) (layer "F.Cu") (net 14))
 (segment (start 98.675 53.7125) (end 100.71 53.7125) (width 0.25) (layer "B.Cu") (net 14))
 (segment (start 99.1225 62.92) (end 99.1225 71.175) (width 0.25) (layer "F.Cu") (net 3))
 (segment (start 99.1225 71.175) (end 100.71 72.7625) (width 0.25) (layer "F.Cu") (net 3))
 (segment (start 100.71 72.7625) (end 98.675 72.7625) (width 0.25) (layer "B.Cu") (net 3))
 (segment (start 99.130471 90.232971) (end 100.71 91.8125) (width 0.25) (layer "F.Cu") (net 31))
 (segment (start 99.130471 81.97) (end 99.130471 90.232971) (width 0.25) (layer "F.Cu") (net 31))
 (segment (start 100.71 91.8125) (end 98.675 91.8125) (width 0.25) (layer "B.Cu") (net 31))
 (segment (start 118.1725 52.125) (end 119.76 53.7125) (width 0.25) (layer "F.Cu") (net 32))
 (segment (start 118.1725 43.87) (end 118.1725 52.125) (width 0.25) (layer "F.Cu") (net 32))
 (segment (start 117.725 53.7125) (end 119.76 53.7125) (width 0.25) (layer "B.Cu") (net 32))
 (segment (start 118.1725 71.175) (end 119.76 72.7625) (width 0.25) (layer "F.Cu") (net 2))
 (segment (start 118.1725 62.92) (end 118.1725 71.175) (width 0.25) (layer "F.Cu") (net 2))
 (segment (start 117.725 72.7625) (end 119.76 72.7625) (width 0.25) (layer "B.Cu") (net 2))
 (segment (start 118.17789 90.23039) (end 119.76 91.8125) (width 0.25) (layer "F.Cu") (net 12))
 (segment (start 118.17789 81.97) (end 118.17789 90.23039) (width 0.25) (layer "F.Cu") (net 12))
 (segment (start 117.725 91.8125) (end 119.76 91.8125) (width 0.25) (layer "B.Cu") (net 12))
 (segment (start 61.62 48.11) (end 57.25 52.48) (width 0.25) (layer "B.Cu") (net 4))
 (segment (start 57.25 52.48) (end 57.25 76.05) (width 0.25) (layer "B.Cu") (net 4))
 (segment (start 55.775 80.8125) (end 57.81 80.8125) (width 0.25) (layer "B.Cu") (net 5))
 (segment (start 57.81 80.8125) (end 53.0475 76.05) (width 0.5) (layer "B.Cu") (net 5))
 (segment (start 53.0475 76.05) (end 50.75 76.05) (width 0.5) (layer "B.Cu") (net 5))
 (segment (start 74.04 72.7625) (end 74.04 68.133743) (width 0.25) (layer "F.Cu") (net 20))
 (segment (start 74.04 68.133743) (end 76 66.173743) (width 0.25) (layer "F.Cu") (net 20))
 (segment (start 74 90) (end 74 87.223743) (width 0.25) (layer "F.Cu") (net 20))
 (segment (start 76 66.173743) (end 76 55.6725) (width 0.25) (layer "F.Cu") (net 20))
 (segment (start 76 55.6725) (end 74.04 53.7125) (width 0.25) (layer "F.Cu") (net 20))
 (segment (start 74 87.223743) (end 75.2975 85.926243) (width 0.25) (layer "F.Cu") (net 20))
 (segment (start 75.2975 85.926243) (end 75.2975 74.02) (width 0.25) (layer "F.Cu") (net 20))
 (segment (start 75.2975 74.02) (end 74.04 72.7625) (width 0.25) (layer "F.Cu") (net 20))
 (via (at 74 90) (size 0.6) (drill 0.3) (layers "F.Cu" "B.Cu") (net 20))
 (segment (start 48.725 65.695) (end 48.725 81.725) (width 0.25) (layer "B.Cu") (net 20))
 (segment (start 74.04 90.04) (end 74 90) (width 0.25) (layer "B.Cu") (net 20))
 (segment (start 74.04 91.8125) (end 74.04 90.04) (width 0.25) (layer "B.Cu") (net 20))
 (segment (start 48.725 81.725) (end 58.8125 91.8125) (width 0.25) (layer "B.Cu") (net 20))
 (segment (start 76.075 72.7625) (end 74.04 72.7625) (width 0.25) (layer "B.Cu") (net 20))
 (segment (start 76.075 91.8125) (end 74.04 91.8125) (width 0.25) (layer "B.Cu") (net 20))
 (segment (start 46.38 63.35) (end 48.725 65.695) (width 0.25) (layer "B.Cu") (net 20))
 (segment (start 58.8125 91.8125) (end 74.04 91.8125) (width 0.25) (layer "B.Cu") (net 20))
 (segment (start 76.075 53.7125) (end 74.04 53.7125) (width 0.25) (layer "B.Cu") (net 20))
 (segment (start 95 66.223743) (end 95 55.6225) (width 0.25) (layer "F.Cu") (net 13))
 (segment (start 93.09 72.7625) (end 93.09 68.133743) (width 0.25) (layer "F.Cu") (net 13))
 (segment (start 94.355471 85.926243) (end 94.355471 74.027971) (width 0.25) (layer "F.Cu") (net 13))
 (segment (start 93.09 68.133743) (end 95 66.223743) (width 0.25) (layer "F.Cu") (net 13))
 (segment (start 95 55.6225) (end 93.09 53.7125) (width 0.25) (layer "F.Cu") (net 13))
 (segment (start 93 87.281714) (end 94.355471 85.926243) (width 0.25) (layer "F.Cu") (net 13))
 (segment (start 94.355471 74.027971) (end 93.09 72.7625) (width 0.25) (layer "F.Cu") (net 13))
 (segment (start 93 90) (end 93 87.281714) (width 0.25) (layer "F.Cu") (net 13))
 (via (at 93 90) (size 0.6) (drill 0.3) (layers "F.Cu" "B.Cu") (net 13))
 (segment (start 45.1787 62.0113) (end 45.1787 79.133888) (width 0.25) (layer "B.Cu") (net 13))
 (segment (start 93.09 90.09) (end 93 90) (width 0.25) (layer "B.Cu") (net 13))
 (segment (start 93.09 53.7125) (end 95.125 53.7125) (width 0.25) (layer "B.Cu") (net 13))
 (segment (start 95.125 72.7625) (end 93.09 72.7625) (width 0.25) (layer "B.Cu") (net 13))
 (segment (start 93.09 91.8125) (end 93.09 90.09) (width 0.25) (layer "B.Cu") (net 13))
 (segment (start 93.09 91.8125) (end 95.125 91.8125) (width 0.25) (layer "B.Cu") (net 13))
 (segment (start 59.044812 93) (end 91.9025 93) (width 0.25) (layer "B.Cu") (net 13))
 (segment (start 46.38 60.81) (end 45.1787 62.0113) (width 0.25) (layer "B.Cu") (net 13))
 (segment (start 45.1787 79.133888) (end 59.044812 93) (width 0.25) (layer "B.Cu") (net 13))
 (segment (start 91.9025 93) (end 93.09 91.8125) (width 0.25) (layer "B.Cu") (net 13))
 (segment (start 113.40289 86.078833) (end 113.40289 74.02539) (width 0.25) (layer "F.Cu") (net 9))
 (segment (start 112 87.481723) (end 113.40289 86.078833) (width 0.25) (layer "F.Cu") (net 9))
 (segment (start 112 90) (end 112 87.481723) (width 0.25) (layer "F.Cu") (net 9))
 (segment (start 114 66.273743) (end 114 55.5725) (width 0.25) (layer "F.Cu") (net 9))
 (segment (start 112.14 68.133743) (end 114 66.273743) (width 0.25) (layer "F.Cu") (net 9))
 (segment (start 113.40289 74.02539) (end 112.14 72.7625) (width 0.25) (layer "F.Cu") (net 9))
 (segment (start 112.14 72.7625) (end 112.14 68.133743) (width 0.25) (layer "F.Cu") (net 9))
 (segment (start 114 55.5725) (end 112.14 53.7125) (width 0.25) (layer "F.Cu") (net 9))
 (via (at 112 90) (size 0.6) (drill 0.3) (layers "F.Cu" "B.Cu") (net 9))
 (segment (start 44.7287 59.9213) (end 44.7287 79.7287) (width 0.25) (layer "B.Cu") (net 9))
 (segment (start 46.38 58.27) (end 44.7287 59.9213) (width 0.25) (layer "B.Cu") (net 9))
 (segment (start 112.14 91.8125) (end 114.175 91.8125) (width 0.25) (layer "B.Cu") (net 9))
 (segment (start 112.14 72.7625) (end 114.175 72.7625) (width 0.25) (layer "B.Cu") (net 9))
 (segment (start 110.5025 93.45) (end 112.14 91.8125) (width 0.25) (layer "B.Cu") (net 9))
 (segment (start 112.14 90.14) (end 112 90) (width 0.25) (layer "B.Cu") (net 9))
 (segment (start 44.7287 79.7287) (end 58.45 93.45) (width 0.25) (layer "B.Cu") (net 9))
 (segment (start 58.45 93.45) (end 110.5025 93.45) (width 0.25) (layer "B.Cu") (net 9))
 (segment (start 114.175 53.7125) (end 112.14 53.7125) (width 0.25) (layer "B.Cu") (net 9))
 (segment (start 112.14 91.8125) (end 112.14 90.14) (width 0.25) (layer "B.Cu") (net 9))
 (segment (start 46.38 48.11) (end 46.38 50.65) (width 0.5) (layer "B.Cu") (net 17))
 (segment (start 49.3 53.57) (end 49.3 79.9225) (width 0.5) (layer "B.Cu") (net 17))
 (segment (start 47.5937 46.8963) (end 46.38 48.11) (width 0.5) (layer "B.Cu") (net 17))
 (segment (start 50.19 80.8125) (end 52.225 80.8125) (width 0.5) (layer "B.Cu") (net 17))
 (segment (start 46.38 50.65) (end 49.3 53.57) (width 0.5) (layer "B.Cu") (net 17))
 (segment (start 49.3 79.9225) (end 50.19 80.8125) (width 0.5) (layer "B.Cu") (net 17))
 (segment (start 60.2937 46.8963) (end 47.5937 46.8963) (width 0.5) (layer "B.Cu") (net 17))
 (segment (start 61.62 45.57) (end 60.2937 46.8963) (width 0.5) (layer "B.Cu") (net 17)))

